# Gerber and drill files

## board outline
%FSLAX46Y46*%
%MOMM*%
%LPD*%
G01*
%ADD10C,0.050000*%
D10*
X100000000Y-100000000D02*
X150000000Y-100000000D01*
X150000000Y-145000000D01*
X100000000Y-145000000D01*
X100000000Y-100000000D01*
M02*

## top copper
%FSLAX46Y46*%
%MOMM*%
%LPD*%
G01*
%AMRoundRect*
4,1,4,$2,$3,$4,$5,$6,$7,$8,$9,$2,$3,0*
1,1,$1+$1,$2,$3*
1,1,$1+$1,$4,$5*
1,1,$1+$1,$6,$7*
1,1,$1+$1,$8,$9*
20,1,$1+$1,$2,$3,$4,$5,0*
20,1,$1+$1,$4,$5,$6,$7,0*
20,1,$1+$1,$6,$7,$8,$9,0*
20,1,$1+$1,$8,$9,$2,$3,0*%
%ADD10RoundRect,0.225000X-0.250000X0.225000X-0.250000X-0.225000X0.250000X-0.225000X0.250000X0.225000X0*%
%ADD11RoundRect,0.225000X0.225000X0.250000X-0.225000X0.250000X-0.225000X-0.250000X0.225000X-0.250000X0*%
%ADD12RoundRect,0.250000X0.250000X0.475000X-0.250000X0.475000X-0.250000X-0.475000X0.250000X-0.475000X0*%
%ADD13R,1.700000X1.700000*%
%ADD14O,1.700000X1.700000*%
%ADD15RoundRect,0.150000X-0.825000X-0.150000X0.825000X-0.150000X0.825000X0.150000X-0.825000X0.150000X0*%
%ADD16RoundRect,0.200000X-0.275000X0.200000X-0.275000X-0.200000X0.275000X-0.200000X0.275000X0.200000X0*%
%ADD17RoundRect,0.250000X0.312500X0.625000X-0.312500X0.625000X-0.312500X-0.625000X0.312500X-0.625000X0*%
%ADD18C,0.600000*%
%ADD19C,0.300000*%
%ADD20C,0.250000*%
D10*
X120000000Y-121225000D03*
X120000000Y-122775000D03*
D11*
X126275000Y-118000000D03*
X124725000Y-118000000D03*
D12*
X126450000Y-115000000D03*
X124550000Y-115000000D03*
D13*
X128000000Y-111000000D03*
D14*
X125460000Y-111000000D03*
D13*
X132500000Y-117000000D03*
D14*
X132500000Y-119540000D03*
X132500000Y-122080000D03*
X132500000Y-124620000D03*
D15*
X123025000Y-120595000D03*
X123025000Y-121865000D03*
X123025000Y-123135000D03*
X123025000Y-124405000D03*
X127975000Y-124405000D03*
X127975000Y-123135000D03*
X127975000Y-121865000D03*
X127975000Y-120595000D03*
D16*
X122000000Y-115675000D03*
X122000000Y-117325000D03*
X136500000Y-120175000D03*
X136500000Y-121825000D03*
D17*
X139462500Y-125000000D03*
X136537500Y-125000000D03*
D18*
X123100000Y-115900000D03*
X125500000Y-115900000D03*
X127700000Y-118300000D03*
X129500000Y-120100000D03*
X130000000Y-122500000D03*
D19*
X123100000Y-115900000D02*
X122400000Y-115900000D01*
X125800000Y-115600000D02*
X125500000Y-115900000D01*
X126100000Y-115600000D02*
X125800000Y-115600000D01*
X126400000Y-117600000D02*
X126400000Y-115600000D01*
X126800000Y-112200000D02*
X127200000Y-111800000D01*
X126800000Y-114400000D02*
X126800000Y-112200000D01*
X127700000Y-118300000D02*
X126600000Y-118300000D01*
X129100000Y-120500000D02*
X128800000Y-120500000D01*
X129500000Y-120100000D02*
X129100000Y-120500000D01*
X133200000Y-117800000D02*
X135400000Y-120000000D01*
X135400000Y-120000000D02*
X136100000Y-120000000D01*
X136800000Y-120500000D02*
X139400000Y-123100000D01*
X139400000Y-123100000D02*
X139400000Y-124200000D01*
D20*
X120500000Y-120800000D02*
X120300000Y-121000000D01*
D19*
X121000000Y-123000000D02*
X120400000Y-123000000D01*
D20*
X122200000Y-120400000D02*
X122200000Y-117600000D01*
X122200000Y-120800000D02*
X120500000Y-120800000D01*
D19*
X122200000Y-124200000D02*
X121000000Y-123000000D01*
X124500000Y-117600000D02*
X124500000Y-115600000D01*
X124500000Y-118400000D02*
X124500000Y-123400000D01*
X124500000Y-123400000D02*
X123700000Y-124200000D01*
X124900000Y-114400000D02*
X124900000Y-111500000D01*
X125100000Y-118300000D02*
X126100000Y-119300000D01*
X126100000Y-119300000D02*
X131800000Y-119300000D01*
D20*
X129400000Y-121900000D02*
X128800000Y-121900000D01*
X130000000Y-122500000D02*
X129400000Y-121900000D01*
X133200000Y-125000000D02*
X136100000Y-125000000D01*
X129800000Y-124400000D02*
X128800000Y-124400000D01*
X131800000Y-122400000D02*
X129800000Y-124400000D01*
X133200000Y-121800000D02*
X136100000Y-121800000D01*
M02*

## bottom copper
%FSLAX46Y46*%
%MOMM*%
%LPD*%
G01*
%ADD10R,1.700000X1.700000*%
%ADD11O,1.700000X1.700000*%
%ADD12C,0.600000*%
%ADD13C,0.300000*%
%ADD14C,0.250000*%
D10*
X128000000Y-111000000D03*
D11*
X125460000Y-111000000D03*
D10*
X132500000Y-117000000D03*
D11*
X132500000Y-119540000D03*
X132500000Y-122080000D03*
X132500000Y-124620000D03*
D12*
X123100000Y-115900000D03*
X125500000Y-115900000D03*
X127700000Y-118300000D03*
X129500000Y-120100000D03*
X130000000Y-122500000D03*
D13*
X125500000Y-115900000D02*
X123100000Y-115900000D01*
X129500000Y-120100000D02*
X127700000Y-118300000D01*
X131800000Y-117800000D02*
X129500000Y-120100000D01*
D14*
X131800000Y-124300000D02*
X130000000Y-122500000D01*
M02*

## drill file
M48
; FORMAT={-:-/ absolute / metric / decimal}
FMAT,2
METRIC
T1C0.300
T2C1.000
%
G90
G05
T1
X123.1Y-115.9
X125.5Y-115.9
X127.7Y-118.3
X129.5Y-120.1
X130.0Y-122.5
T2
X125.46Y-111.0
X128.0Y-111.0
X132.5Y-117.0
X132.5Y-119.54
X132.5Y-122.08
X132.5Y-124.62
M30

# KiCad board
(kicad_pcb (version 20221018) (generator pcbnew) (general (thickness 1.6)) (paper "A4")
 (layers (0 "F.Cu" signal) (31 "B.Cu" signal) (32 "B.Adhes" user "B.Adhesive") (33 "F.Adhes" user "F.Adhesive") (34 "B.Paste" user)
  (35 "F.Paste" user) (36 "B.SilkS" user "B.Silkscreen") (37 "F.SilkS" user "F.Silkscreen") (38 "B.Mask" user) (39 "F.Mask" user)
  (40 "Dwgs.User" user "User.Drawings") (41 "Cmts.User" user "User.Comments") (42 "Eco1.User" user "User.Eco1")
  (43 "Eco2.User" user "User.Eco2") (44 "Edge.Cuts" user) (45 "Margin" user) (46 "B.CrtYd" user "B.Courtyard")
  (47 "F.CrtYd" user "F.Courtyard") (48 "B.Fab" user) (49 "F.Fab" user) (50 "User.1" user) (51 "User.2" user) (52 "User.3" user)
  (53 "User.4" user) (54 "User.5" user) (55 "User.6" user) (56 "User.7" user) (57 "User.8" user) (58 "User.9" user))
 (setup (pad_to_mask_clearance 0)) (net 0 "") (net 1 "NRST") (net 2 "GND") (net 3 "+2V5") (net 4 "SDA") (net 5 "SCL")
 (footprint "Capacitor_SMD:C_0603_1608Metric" (layer "F.Cu") (at 120 122 -90)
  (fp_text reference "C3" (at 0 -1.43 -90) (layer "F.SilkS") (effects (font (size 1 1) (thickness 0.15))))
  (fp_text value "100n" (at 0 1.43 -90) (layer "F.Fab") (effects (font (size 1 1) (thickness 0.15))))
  (pad "1" smd roundrect (at -0.775 0 270) (size 0.9 0.95) (layers "F.Cu" "F.Paste" "F.Mask") (roundrect_rratio 0.25) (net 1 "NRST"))
  (pad "2" smd roundrect (at 0.775 0 270) (size 0.9 0.95) (layers "F.Cu" "F.Paste" "F.Mask") (roundrect_rratio 0.25) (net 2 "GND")))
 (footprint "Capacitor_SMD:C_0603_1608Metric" (layer "F.Cu") (at 125.5 118 180)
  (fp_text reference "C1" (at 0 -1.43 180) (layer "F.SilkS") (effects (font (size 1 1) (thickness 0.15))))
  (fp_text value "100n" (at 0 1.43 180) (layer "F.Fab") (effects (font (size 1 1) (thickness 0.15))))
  (pad "1" smd roundrect (at -0.775 0 180) (size 0.9 0.95) (layers "F.Cu" "F.Paste" "F.Mask") (roundrect_rratio 0.25) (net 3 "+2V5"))
  (pad "2" smd roundrect (at 0.775 0 180) (size 0.9 0.95) (layers "F.Cu" "F.Paste" "F.Mask") (roundrect_rratio 0.25) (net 2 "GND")))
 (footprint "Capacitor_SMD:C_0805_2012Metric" (layer "F.Cu") (at 125.5 115 180)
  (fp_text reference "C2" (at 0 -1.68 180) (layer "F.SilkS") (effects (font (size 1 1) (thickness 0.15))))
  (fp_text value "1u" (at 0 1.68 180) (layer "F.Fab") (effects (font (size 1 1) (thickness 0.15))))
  (pad "1" smd roundrect (at -0.95 0 180) (size 1 1.45) (layers "F.Cu" "F.Paste" "F.Mask") (roundrect_rratio 0.25) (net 3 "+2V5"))
  (pad "2" smd roundrect (at 0.95 0 180) (size 1 1.45) (layers "F.Cu" "F.Paste" "F.Mask") (roundrect_rratio 0.25) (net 2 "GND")))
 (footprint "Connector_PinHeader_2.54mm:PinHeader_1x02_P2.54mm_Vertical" (layer "F.Cu") (at 128 111 -90)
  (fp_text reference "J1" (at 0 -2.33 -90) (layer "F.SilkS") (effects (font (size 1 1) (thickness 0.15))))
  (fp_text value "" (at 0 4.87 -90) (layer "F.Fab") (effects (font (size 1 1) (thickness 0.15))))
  (pad "1" thru_hole rect (at 0 0 270) (size 1.7 1.7) (drill 1) (layers "*.Cu" "*.Mask") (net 3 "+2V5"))
  (pad "2" thru_hole oval (at 0 2.54 270) (size 1.7 1.7) (drill 1) (layers "*.Cu" "*.Mask") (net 2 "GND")))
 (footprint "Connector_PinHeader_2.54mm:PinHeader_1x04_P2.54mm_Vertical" (layer "F.Cu") (at 132.5 117)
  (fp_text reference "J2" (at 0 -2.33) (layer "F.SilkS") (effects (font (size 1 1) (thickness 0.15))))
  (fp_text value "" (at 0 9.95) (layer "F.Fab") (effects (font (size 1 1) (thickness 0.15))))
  (pad "1" thru_hole rect (at 0 0) (size 1.7 1.7) (drill 1) (layers "*.Cu" "*.Mask") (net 3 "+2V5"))
  (pad "2" thru_hole oval (at 0 2.54) (size 1.7 1.7) (drill 1) (layers "*.Cu" "*.Mask") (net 2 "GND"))
  (pad "3" thru_hole oval (at 0 5.08) (size 1.7 1.7) (drill 1) (layers "*.Cu" "*.Mask") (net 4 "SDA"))
  (pad "4" thru_hole oval (at 0 7.62) (size 1.7 1.7) (drill 1) (layers "*.Cu" "*.Mask") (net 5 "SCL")))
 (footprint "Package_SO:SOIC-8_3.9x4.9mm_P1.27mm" (layer "F.Cu") (at 125.5 122.5)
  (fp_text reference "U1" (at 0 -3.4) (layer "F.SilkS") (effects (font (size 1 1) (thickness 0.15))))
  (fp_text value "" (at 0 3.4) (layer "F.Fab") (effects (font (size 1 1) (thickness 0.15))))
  (pad "1" smd roundrect (at -2.475 -1.905) (size 1.95 0.6) (layers "F.Cu" "F.Paste" "F.Mask") (roundrect_rratio 0.25) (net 1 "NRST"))
  (pad "2" smd roundrect (at -2.475 -0.635) (size 1.95 0.6) (layers "F.Cu" "F.Paste" "F.Mask") (roundrect_rratio 0.25))
  (pad "3" smd roundrect (at -2.475 0.635) (size 1.95 0.6) (layers "F.Cu" "F.Paste" "F.Mask") (roundrect_rratio 0.25))
  (pad "4" smd roundrect (at -2.475 1.905) (size 1.95 0.6) (layers "F.Cu" "F.Paste" "F.Mask") (roundrect_rratio 0.25) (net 2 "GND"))
  (pad "5" smd roundrect (at 2.475 1.905) (size 1.95 0.6) (layers "F.Cu" "F.Paste" "F.Mask") (roundrect_rratio 0.25) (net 4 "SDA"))
  (pad "6" smd roundrect (at 2.475 0.635) (size 1.95 0.6) (layers "F.Cu" "F.Paste" "F.Mask") (roundrect_rratio 0.25))
  (pad "7" smd roundrect (at 2.475 -0.635) (size 1.95 0.6) (layers "F.Cu" "F.Paste" "F.Mask") (roundrect_rratio 0.25) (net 5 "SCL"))
  (pad "8" smd roundrect (at 2.475 -1.905) (size 1.95 0.6) (layers "F.Cu" "F.Paste" "F.Mask") (roundrect_rratio 0.25) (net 3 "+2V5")))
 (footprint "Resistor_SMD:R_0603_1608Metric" (layer "F.Cu") (at 122 116.5 -90)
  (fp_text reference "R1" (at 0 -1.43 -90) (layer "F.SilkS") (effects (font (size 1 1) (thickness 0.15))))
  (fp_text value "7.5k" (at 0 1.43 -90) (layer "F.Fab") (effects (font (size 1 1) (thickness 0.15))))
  (pad "1" smd roundrect (at -0.825 0 270) (size 0.8 0.95) (layers "F.Cu" "F.Paste" "F.Mask") (roundrect_rratio 0.25) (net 3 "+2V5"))
  (pad "2" smd roundrect (at 0.825 0 270) (size 0.8 0.95) (layers "F.Cu" "F.Paste" "F.Mask") (roundrect_rratio 0.25) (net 1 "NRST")))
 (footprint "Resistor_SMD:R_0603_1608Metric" (layer "F.Cu") (at 136.5 121 -90)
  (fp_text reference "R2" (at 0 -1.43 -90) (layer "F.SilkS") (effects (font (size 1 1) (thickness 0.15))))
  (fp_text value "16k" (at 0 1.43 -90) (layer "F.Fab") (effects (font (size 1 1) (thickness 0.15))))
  (pad "1" smd roundrect (at -0.825 0 270) (size 0.8 0.95) (layers "F.Cu" "F.Paste" "F.Mask") (roundrect_rratio 0.25) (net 3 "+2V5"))
  (pad "2" smd roundrect (at 0.825 0 270) (size 0.8 0.95) (layers "F.Cu" "F.Paste" "F.Mask") (roundrect_rratio 0.25) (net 4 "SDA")))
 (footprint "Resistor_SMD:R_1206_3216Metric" (layer "F.Cu") (at 138 125 180)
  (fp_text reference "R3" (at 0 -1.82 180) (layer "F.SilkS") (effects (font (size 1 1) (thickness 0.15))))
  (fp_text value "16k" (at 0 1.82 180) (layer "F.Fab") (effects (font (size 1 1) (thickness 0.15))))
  (pad "1" smd roundrect (at -1.4625 0 180) (size 1.125 1.75) (layers "F.Cu" "F.Paste" "F.Mask") (roundrect_rratio 0.222222) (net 3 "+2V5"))
  (pad "2" smd roundrect (at 1.4625 0 180) (size 1.125 1.75) (layers "F.Cu" "F.Paste" "F.Mask") (roundrect_rratio 0.222222) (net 5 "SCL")))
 (gr_rect (start 100 100) (end 150 145) (stroke (width 0.05) (type default)) (fill none) (layer "Edge.Cuts"))
 (segment (start 123.1 115.9) (end 122.4 115.9) (width 0.3) (layer "F.Cu") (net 3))
 (segment (start 125.8 115.6) (end 125.5 115.9) (width 0.3) (layer "F.Cu") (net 3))
 (segment (start 126.1 115.6) (end 125.8 115.6) (width 0.3) (layer "F.Cu") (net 3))
 (segment (start 126.4 117.6) (end 126.4 115.6) (width 0.3) (layer "F.Cu") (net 3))
 (segment (start 126.8 112.2) (end 127.2 111.8) (width 0.3) (layer "F.Cu") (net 3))
 (segment (start 126.8 114.4) (end 126.8 112.2) (width 0.3) (layer "F.Cu") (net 3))
 (segment (start 127.7 118.3) (end 126.6 118.3) (width 0.3) (layer "F.Cu") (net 3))
 (segment (start 129.1 120.5) (end 128.8 120.5) (width 0.3) (layer "F.Cu") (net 3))
 (segment (start 129.5 120.1) (end 129.1 120.5) (width 0.3) (layer "F.Cu") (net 3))
 (segment (start 133.2 117.8) (end 135.4 120) (width 0.3) (layer "F.Cu") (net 3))
 (segment (start 135.4 120) (end 136.1 120) (width 0.3) (layer "F.Cu") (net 3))
 (segment (start 136.8 120.5) (end 139.4 123.1) (width 0.3) (layer "F.Cu") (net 3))
 (segment (start 139.4 123.1) (end 139.4 124.2) (width 0.3) (layer "F.Cu") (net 3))
 (via (at 123.1 115.9) (size 0.6) (drill 0.3) (layers "F.Cu" "B.Cu") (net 3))
 (via (at 125.5 115.9) (size 0.6) (drill 0.3) (layers "F.Cu" "B.Cu") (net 3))
 (via (at 127.7 118.3) (size 0.6) (drill 0.3) (layers "F.Cu" "B.Cu") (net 3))
 (via (at 129.5 120.1) (size 0.6) (drill 0.3) (layers "F.Cu" "B.Cu") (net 3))
 (segment (start 120.5 120.8) (end 120.3 121) (width 0.25) (layer "F.Cu") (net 1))
 (segment (start 121 123) (end 120.4 123) (width 0.3) (layer "F.Cu") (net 2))
 (segment (start 122.2 120.4) (end 122.2 117.6) (width 0.25) (layer "F.Cu") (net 1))
 (segment (start 122.2 120.8) (end 120.5 120.8) (width 0.25) (layer "F.Cu") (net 1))
 (segment (start 122.2 124.2) (end 121 123) (width 0.3) (layer "F.Cu") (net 2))
 (segment (start 124.5 117.6) (end 124.5 115.6) (width 0.3) (layer "F.Cu") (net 2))
 (segment (start 124.5 118.4) (end 124.5 123.4) (width 0.3) (layer "F.Cu") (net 2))
 (segment (start 124.5 123.4) (end 123.7 124.2) (width 0.3) (layer "F.Cu") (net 2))
 (segment (start 124.9 114.4) (end 124.9 111.5) (width 0.3) (layer "F.Cu") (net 2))
 (segment (start 125.1 118.3) (end 126.1 119.3) (width 0.3) (layer "F.Cu") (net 2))
 (segment (start 125.5 115.9) (end 123.1 115.9) (width 0.3) (layer "B.Cu") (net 3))
 (segment (start 126.1 119.3) (end 131.8 119.3) (width 0.3) (layer "F.Cu") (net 2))
 (segment (start 129.4 121.9) (end 128.8 121.9) (width 0.25) (layer "F.Cu") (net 5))
 (segment (start 129.5 120.1) (end 127.7 118.3) (width 0.3) (layer "B.Cu") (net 3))
 (segment (start 130 122.5) (end 129.4 121.9) (width 0.25) (layer "F.Cu") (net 5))
 (segment (start 131.8 117.8) (end 129.5 120.1) (width 0.3) (layer "B.Cu") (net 3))
 (segment (start 133.2 125) (end 136.1 125) (width 0.25) (layer "F.Cu") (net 5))
 (via (at 130 122.5) (size 0.6) (drill 0.3) (layers "F.Cu" "B.Cu") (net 5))
 (segment (start 129.8 124.4) (end 128.8 124.4) (width 0.25) (layer "F.Cu") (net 4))
 (segment (start 131.8 122.4) (end 129.8 124.4) (width 0.25) (layer "F.Cu") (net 4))
 (segment (start 131.8 124.3) (end 130 122.5) (width 0.25) (layer "B.Cu") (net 5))
 (segment (start 133.2 121.8) (end 136.1 121.8) (width 0.25) (layer "F.Cu") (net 4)))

